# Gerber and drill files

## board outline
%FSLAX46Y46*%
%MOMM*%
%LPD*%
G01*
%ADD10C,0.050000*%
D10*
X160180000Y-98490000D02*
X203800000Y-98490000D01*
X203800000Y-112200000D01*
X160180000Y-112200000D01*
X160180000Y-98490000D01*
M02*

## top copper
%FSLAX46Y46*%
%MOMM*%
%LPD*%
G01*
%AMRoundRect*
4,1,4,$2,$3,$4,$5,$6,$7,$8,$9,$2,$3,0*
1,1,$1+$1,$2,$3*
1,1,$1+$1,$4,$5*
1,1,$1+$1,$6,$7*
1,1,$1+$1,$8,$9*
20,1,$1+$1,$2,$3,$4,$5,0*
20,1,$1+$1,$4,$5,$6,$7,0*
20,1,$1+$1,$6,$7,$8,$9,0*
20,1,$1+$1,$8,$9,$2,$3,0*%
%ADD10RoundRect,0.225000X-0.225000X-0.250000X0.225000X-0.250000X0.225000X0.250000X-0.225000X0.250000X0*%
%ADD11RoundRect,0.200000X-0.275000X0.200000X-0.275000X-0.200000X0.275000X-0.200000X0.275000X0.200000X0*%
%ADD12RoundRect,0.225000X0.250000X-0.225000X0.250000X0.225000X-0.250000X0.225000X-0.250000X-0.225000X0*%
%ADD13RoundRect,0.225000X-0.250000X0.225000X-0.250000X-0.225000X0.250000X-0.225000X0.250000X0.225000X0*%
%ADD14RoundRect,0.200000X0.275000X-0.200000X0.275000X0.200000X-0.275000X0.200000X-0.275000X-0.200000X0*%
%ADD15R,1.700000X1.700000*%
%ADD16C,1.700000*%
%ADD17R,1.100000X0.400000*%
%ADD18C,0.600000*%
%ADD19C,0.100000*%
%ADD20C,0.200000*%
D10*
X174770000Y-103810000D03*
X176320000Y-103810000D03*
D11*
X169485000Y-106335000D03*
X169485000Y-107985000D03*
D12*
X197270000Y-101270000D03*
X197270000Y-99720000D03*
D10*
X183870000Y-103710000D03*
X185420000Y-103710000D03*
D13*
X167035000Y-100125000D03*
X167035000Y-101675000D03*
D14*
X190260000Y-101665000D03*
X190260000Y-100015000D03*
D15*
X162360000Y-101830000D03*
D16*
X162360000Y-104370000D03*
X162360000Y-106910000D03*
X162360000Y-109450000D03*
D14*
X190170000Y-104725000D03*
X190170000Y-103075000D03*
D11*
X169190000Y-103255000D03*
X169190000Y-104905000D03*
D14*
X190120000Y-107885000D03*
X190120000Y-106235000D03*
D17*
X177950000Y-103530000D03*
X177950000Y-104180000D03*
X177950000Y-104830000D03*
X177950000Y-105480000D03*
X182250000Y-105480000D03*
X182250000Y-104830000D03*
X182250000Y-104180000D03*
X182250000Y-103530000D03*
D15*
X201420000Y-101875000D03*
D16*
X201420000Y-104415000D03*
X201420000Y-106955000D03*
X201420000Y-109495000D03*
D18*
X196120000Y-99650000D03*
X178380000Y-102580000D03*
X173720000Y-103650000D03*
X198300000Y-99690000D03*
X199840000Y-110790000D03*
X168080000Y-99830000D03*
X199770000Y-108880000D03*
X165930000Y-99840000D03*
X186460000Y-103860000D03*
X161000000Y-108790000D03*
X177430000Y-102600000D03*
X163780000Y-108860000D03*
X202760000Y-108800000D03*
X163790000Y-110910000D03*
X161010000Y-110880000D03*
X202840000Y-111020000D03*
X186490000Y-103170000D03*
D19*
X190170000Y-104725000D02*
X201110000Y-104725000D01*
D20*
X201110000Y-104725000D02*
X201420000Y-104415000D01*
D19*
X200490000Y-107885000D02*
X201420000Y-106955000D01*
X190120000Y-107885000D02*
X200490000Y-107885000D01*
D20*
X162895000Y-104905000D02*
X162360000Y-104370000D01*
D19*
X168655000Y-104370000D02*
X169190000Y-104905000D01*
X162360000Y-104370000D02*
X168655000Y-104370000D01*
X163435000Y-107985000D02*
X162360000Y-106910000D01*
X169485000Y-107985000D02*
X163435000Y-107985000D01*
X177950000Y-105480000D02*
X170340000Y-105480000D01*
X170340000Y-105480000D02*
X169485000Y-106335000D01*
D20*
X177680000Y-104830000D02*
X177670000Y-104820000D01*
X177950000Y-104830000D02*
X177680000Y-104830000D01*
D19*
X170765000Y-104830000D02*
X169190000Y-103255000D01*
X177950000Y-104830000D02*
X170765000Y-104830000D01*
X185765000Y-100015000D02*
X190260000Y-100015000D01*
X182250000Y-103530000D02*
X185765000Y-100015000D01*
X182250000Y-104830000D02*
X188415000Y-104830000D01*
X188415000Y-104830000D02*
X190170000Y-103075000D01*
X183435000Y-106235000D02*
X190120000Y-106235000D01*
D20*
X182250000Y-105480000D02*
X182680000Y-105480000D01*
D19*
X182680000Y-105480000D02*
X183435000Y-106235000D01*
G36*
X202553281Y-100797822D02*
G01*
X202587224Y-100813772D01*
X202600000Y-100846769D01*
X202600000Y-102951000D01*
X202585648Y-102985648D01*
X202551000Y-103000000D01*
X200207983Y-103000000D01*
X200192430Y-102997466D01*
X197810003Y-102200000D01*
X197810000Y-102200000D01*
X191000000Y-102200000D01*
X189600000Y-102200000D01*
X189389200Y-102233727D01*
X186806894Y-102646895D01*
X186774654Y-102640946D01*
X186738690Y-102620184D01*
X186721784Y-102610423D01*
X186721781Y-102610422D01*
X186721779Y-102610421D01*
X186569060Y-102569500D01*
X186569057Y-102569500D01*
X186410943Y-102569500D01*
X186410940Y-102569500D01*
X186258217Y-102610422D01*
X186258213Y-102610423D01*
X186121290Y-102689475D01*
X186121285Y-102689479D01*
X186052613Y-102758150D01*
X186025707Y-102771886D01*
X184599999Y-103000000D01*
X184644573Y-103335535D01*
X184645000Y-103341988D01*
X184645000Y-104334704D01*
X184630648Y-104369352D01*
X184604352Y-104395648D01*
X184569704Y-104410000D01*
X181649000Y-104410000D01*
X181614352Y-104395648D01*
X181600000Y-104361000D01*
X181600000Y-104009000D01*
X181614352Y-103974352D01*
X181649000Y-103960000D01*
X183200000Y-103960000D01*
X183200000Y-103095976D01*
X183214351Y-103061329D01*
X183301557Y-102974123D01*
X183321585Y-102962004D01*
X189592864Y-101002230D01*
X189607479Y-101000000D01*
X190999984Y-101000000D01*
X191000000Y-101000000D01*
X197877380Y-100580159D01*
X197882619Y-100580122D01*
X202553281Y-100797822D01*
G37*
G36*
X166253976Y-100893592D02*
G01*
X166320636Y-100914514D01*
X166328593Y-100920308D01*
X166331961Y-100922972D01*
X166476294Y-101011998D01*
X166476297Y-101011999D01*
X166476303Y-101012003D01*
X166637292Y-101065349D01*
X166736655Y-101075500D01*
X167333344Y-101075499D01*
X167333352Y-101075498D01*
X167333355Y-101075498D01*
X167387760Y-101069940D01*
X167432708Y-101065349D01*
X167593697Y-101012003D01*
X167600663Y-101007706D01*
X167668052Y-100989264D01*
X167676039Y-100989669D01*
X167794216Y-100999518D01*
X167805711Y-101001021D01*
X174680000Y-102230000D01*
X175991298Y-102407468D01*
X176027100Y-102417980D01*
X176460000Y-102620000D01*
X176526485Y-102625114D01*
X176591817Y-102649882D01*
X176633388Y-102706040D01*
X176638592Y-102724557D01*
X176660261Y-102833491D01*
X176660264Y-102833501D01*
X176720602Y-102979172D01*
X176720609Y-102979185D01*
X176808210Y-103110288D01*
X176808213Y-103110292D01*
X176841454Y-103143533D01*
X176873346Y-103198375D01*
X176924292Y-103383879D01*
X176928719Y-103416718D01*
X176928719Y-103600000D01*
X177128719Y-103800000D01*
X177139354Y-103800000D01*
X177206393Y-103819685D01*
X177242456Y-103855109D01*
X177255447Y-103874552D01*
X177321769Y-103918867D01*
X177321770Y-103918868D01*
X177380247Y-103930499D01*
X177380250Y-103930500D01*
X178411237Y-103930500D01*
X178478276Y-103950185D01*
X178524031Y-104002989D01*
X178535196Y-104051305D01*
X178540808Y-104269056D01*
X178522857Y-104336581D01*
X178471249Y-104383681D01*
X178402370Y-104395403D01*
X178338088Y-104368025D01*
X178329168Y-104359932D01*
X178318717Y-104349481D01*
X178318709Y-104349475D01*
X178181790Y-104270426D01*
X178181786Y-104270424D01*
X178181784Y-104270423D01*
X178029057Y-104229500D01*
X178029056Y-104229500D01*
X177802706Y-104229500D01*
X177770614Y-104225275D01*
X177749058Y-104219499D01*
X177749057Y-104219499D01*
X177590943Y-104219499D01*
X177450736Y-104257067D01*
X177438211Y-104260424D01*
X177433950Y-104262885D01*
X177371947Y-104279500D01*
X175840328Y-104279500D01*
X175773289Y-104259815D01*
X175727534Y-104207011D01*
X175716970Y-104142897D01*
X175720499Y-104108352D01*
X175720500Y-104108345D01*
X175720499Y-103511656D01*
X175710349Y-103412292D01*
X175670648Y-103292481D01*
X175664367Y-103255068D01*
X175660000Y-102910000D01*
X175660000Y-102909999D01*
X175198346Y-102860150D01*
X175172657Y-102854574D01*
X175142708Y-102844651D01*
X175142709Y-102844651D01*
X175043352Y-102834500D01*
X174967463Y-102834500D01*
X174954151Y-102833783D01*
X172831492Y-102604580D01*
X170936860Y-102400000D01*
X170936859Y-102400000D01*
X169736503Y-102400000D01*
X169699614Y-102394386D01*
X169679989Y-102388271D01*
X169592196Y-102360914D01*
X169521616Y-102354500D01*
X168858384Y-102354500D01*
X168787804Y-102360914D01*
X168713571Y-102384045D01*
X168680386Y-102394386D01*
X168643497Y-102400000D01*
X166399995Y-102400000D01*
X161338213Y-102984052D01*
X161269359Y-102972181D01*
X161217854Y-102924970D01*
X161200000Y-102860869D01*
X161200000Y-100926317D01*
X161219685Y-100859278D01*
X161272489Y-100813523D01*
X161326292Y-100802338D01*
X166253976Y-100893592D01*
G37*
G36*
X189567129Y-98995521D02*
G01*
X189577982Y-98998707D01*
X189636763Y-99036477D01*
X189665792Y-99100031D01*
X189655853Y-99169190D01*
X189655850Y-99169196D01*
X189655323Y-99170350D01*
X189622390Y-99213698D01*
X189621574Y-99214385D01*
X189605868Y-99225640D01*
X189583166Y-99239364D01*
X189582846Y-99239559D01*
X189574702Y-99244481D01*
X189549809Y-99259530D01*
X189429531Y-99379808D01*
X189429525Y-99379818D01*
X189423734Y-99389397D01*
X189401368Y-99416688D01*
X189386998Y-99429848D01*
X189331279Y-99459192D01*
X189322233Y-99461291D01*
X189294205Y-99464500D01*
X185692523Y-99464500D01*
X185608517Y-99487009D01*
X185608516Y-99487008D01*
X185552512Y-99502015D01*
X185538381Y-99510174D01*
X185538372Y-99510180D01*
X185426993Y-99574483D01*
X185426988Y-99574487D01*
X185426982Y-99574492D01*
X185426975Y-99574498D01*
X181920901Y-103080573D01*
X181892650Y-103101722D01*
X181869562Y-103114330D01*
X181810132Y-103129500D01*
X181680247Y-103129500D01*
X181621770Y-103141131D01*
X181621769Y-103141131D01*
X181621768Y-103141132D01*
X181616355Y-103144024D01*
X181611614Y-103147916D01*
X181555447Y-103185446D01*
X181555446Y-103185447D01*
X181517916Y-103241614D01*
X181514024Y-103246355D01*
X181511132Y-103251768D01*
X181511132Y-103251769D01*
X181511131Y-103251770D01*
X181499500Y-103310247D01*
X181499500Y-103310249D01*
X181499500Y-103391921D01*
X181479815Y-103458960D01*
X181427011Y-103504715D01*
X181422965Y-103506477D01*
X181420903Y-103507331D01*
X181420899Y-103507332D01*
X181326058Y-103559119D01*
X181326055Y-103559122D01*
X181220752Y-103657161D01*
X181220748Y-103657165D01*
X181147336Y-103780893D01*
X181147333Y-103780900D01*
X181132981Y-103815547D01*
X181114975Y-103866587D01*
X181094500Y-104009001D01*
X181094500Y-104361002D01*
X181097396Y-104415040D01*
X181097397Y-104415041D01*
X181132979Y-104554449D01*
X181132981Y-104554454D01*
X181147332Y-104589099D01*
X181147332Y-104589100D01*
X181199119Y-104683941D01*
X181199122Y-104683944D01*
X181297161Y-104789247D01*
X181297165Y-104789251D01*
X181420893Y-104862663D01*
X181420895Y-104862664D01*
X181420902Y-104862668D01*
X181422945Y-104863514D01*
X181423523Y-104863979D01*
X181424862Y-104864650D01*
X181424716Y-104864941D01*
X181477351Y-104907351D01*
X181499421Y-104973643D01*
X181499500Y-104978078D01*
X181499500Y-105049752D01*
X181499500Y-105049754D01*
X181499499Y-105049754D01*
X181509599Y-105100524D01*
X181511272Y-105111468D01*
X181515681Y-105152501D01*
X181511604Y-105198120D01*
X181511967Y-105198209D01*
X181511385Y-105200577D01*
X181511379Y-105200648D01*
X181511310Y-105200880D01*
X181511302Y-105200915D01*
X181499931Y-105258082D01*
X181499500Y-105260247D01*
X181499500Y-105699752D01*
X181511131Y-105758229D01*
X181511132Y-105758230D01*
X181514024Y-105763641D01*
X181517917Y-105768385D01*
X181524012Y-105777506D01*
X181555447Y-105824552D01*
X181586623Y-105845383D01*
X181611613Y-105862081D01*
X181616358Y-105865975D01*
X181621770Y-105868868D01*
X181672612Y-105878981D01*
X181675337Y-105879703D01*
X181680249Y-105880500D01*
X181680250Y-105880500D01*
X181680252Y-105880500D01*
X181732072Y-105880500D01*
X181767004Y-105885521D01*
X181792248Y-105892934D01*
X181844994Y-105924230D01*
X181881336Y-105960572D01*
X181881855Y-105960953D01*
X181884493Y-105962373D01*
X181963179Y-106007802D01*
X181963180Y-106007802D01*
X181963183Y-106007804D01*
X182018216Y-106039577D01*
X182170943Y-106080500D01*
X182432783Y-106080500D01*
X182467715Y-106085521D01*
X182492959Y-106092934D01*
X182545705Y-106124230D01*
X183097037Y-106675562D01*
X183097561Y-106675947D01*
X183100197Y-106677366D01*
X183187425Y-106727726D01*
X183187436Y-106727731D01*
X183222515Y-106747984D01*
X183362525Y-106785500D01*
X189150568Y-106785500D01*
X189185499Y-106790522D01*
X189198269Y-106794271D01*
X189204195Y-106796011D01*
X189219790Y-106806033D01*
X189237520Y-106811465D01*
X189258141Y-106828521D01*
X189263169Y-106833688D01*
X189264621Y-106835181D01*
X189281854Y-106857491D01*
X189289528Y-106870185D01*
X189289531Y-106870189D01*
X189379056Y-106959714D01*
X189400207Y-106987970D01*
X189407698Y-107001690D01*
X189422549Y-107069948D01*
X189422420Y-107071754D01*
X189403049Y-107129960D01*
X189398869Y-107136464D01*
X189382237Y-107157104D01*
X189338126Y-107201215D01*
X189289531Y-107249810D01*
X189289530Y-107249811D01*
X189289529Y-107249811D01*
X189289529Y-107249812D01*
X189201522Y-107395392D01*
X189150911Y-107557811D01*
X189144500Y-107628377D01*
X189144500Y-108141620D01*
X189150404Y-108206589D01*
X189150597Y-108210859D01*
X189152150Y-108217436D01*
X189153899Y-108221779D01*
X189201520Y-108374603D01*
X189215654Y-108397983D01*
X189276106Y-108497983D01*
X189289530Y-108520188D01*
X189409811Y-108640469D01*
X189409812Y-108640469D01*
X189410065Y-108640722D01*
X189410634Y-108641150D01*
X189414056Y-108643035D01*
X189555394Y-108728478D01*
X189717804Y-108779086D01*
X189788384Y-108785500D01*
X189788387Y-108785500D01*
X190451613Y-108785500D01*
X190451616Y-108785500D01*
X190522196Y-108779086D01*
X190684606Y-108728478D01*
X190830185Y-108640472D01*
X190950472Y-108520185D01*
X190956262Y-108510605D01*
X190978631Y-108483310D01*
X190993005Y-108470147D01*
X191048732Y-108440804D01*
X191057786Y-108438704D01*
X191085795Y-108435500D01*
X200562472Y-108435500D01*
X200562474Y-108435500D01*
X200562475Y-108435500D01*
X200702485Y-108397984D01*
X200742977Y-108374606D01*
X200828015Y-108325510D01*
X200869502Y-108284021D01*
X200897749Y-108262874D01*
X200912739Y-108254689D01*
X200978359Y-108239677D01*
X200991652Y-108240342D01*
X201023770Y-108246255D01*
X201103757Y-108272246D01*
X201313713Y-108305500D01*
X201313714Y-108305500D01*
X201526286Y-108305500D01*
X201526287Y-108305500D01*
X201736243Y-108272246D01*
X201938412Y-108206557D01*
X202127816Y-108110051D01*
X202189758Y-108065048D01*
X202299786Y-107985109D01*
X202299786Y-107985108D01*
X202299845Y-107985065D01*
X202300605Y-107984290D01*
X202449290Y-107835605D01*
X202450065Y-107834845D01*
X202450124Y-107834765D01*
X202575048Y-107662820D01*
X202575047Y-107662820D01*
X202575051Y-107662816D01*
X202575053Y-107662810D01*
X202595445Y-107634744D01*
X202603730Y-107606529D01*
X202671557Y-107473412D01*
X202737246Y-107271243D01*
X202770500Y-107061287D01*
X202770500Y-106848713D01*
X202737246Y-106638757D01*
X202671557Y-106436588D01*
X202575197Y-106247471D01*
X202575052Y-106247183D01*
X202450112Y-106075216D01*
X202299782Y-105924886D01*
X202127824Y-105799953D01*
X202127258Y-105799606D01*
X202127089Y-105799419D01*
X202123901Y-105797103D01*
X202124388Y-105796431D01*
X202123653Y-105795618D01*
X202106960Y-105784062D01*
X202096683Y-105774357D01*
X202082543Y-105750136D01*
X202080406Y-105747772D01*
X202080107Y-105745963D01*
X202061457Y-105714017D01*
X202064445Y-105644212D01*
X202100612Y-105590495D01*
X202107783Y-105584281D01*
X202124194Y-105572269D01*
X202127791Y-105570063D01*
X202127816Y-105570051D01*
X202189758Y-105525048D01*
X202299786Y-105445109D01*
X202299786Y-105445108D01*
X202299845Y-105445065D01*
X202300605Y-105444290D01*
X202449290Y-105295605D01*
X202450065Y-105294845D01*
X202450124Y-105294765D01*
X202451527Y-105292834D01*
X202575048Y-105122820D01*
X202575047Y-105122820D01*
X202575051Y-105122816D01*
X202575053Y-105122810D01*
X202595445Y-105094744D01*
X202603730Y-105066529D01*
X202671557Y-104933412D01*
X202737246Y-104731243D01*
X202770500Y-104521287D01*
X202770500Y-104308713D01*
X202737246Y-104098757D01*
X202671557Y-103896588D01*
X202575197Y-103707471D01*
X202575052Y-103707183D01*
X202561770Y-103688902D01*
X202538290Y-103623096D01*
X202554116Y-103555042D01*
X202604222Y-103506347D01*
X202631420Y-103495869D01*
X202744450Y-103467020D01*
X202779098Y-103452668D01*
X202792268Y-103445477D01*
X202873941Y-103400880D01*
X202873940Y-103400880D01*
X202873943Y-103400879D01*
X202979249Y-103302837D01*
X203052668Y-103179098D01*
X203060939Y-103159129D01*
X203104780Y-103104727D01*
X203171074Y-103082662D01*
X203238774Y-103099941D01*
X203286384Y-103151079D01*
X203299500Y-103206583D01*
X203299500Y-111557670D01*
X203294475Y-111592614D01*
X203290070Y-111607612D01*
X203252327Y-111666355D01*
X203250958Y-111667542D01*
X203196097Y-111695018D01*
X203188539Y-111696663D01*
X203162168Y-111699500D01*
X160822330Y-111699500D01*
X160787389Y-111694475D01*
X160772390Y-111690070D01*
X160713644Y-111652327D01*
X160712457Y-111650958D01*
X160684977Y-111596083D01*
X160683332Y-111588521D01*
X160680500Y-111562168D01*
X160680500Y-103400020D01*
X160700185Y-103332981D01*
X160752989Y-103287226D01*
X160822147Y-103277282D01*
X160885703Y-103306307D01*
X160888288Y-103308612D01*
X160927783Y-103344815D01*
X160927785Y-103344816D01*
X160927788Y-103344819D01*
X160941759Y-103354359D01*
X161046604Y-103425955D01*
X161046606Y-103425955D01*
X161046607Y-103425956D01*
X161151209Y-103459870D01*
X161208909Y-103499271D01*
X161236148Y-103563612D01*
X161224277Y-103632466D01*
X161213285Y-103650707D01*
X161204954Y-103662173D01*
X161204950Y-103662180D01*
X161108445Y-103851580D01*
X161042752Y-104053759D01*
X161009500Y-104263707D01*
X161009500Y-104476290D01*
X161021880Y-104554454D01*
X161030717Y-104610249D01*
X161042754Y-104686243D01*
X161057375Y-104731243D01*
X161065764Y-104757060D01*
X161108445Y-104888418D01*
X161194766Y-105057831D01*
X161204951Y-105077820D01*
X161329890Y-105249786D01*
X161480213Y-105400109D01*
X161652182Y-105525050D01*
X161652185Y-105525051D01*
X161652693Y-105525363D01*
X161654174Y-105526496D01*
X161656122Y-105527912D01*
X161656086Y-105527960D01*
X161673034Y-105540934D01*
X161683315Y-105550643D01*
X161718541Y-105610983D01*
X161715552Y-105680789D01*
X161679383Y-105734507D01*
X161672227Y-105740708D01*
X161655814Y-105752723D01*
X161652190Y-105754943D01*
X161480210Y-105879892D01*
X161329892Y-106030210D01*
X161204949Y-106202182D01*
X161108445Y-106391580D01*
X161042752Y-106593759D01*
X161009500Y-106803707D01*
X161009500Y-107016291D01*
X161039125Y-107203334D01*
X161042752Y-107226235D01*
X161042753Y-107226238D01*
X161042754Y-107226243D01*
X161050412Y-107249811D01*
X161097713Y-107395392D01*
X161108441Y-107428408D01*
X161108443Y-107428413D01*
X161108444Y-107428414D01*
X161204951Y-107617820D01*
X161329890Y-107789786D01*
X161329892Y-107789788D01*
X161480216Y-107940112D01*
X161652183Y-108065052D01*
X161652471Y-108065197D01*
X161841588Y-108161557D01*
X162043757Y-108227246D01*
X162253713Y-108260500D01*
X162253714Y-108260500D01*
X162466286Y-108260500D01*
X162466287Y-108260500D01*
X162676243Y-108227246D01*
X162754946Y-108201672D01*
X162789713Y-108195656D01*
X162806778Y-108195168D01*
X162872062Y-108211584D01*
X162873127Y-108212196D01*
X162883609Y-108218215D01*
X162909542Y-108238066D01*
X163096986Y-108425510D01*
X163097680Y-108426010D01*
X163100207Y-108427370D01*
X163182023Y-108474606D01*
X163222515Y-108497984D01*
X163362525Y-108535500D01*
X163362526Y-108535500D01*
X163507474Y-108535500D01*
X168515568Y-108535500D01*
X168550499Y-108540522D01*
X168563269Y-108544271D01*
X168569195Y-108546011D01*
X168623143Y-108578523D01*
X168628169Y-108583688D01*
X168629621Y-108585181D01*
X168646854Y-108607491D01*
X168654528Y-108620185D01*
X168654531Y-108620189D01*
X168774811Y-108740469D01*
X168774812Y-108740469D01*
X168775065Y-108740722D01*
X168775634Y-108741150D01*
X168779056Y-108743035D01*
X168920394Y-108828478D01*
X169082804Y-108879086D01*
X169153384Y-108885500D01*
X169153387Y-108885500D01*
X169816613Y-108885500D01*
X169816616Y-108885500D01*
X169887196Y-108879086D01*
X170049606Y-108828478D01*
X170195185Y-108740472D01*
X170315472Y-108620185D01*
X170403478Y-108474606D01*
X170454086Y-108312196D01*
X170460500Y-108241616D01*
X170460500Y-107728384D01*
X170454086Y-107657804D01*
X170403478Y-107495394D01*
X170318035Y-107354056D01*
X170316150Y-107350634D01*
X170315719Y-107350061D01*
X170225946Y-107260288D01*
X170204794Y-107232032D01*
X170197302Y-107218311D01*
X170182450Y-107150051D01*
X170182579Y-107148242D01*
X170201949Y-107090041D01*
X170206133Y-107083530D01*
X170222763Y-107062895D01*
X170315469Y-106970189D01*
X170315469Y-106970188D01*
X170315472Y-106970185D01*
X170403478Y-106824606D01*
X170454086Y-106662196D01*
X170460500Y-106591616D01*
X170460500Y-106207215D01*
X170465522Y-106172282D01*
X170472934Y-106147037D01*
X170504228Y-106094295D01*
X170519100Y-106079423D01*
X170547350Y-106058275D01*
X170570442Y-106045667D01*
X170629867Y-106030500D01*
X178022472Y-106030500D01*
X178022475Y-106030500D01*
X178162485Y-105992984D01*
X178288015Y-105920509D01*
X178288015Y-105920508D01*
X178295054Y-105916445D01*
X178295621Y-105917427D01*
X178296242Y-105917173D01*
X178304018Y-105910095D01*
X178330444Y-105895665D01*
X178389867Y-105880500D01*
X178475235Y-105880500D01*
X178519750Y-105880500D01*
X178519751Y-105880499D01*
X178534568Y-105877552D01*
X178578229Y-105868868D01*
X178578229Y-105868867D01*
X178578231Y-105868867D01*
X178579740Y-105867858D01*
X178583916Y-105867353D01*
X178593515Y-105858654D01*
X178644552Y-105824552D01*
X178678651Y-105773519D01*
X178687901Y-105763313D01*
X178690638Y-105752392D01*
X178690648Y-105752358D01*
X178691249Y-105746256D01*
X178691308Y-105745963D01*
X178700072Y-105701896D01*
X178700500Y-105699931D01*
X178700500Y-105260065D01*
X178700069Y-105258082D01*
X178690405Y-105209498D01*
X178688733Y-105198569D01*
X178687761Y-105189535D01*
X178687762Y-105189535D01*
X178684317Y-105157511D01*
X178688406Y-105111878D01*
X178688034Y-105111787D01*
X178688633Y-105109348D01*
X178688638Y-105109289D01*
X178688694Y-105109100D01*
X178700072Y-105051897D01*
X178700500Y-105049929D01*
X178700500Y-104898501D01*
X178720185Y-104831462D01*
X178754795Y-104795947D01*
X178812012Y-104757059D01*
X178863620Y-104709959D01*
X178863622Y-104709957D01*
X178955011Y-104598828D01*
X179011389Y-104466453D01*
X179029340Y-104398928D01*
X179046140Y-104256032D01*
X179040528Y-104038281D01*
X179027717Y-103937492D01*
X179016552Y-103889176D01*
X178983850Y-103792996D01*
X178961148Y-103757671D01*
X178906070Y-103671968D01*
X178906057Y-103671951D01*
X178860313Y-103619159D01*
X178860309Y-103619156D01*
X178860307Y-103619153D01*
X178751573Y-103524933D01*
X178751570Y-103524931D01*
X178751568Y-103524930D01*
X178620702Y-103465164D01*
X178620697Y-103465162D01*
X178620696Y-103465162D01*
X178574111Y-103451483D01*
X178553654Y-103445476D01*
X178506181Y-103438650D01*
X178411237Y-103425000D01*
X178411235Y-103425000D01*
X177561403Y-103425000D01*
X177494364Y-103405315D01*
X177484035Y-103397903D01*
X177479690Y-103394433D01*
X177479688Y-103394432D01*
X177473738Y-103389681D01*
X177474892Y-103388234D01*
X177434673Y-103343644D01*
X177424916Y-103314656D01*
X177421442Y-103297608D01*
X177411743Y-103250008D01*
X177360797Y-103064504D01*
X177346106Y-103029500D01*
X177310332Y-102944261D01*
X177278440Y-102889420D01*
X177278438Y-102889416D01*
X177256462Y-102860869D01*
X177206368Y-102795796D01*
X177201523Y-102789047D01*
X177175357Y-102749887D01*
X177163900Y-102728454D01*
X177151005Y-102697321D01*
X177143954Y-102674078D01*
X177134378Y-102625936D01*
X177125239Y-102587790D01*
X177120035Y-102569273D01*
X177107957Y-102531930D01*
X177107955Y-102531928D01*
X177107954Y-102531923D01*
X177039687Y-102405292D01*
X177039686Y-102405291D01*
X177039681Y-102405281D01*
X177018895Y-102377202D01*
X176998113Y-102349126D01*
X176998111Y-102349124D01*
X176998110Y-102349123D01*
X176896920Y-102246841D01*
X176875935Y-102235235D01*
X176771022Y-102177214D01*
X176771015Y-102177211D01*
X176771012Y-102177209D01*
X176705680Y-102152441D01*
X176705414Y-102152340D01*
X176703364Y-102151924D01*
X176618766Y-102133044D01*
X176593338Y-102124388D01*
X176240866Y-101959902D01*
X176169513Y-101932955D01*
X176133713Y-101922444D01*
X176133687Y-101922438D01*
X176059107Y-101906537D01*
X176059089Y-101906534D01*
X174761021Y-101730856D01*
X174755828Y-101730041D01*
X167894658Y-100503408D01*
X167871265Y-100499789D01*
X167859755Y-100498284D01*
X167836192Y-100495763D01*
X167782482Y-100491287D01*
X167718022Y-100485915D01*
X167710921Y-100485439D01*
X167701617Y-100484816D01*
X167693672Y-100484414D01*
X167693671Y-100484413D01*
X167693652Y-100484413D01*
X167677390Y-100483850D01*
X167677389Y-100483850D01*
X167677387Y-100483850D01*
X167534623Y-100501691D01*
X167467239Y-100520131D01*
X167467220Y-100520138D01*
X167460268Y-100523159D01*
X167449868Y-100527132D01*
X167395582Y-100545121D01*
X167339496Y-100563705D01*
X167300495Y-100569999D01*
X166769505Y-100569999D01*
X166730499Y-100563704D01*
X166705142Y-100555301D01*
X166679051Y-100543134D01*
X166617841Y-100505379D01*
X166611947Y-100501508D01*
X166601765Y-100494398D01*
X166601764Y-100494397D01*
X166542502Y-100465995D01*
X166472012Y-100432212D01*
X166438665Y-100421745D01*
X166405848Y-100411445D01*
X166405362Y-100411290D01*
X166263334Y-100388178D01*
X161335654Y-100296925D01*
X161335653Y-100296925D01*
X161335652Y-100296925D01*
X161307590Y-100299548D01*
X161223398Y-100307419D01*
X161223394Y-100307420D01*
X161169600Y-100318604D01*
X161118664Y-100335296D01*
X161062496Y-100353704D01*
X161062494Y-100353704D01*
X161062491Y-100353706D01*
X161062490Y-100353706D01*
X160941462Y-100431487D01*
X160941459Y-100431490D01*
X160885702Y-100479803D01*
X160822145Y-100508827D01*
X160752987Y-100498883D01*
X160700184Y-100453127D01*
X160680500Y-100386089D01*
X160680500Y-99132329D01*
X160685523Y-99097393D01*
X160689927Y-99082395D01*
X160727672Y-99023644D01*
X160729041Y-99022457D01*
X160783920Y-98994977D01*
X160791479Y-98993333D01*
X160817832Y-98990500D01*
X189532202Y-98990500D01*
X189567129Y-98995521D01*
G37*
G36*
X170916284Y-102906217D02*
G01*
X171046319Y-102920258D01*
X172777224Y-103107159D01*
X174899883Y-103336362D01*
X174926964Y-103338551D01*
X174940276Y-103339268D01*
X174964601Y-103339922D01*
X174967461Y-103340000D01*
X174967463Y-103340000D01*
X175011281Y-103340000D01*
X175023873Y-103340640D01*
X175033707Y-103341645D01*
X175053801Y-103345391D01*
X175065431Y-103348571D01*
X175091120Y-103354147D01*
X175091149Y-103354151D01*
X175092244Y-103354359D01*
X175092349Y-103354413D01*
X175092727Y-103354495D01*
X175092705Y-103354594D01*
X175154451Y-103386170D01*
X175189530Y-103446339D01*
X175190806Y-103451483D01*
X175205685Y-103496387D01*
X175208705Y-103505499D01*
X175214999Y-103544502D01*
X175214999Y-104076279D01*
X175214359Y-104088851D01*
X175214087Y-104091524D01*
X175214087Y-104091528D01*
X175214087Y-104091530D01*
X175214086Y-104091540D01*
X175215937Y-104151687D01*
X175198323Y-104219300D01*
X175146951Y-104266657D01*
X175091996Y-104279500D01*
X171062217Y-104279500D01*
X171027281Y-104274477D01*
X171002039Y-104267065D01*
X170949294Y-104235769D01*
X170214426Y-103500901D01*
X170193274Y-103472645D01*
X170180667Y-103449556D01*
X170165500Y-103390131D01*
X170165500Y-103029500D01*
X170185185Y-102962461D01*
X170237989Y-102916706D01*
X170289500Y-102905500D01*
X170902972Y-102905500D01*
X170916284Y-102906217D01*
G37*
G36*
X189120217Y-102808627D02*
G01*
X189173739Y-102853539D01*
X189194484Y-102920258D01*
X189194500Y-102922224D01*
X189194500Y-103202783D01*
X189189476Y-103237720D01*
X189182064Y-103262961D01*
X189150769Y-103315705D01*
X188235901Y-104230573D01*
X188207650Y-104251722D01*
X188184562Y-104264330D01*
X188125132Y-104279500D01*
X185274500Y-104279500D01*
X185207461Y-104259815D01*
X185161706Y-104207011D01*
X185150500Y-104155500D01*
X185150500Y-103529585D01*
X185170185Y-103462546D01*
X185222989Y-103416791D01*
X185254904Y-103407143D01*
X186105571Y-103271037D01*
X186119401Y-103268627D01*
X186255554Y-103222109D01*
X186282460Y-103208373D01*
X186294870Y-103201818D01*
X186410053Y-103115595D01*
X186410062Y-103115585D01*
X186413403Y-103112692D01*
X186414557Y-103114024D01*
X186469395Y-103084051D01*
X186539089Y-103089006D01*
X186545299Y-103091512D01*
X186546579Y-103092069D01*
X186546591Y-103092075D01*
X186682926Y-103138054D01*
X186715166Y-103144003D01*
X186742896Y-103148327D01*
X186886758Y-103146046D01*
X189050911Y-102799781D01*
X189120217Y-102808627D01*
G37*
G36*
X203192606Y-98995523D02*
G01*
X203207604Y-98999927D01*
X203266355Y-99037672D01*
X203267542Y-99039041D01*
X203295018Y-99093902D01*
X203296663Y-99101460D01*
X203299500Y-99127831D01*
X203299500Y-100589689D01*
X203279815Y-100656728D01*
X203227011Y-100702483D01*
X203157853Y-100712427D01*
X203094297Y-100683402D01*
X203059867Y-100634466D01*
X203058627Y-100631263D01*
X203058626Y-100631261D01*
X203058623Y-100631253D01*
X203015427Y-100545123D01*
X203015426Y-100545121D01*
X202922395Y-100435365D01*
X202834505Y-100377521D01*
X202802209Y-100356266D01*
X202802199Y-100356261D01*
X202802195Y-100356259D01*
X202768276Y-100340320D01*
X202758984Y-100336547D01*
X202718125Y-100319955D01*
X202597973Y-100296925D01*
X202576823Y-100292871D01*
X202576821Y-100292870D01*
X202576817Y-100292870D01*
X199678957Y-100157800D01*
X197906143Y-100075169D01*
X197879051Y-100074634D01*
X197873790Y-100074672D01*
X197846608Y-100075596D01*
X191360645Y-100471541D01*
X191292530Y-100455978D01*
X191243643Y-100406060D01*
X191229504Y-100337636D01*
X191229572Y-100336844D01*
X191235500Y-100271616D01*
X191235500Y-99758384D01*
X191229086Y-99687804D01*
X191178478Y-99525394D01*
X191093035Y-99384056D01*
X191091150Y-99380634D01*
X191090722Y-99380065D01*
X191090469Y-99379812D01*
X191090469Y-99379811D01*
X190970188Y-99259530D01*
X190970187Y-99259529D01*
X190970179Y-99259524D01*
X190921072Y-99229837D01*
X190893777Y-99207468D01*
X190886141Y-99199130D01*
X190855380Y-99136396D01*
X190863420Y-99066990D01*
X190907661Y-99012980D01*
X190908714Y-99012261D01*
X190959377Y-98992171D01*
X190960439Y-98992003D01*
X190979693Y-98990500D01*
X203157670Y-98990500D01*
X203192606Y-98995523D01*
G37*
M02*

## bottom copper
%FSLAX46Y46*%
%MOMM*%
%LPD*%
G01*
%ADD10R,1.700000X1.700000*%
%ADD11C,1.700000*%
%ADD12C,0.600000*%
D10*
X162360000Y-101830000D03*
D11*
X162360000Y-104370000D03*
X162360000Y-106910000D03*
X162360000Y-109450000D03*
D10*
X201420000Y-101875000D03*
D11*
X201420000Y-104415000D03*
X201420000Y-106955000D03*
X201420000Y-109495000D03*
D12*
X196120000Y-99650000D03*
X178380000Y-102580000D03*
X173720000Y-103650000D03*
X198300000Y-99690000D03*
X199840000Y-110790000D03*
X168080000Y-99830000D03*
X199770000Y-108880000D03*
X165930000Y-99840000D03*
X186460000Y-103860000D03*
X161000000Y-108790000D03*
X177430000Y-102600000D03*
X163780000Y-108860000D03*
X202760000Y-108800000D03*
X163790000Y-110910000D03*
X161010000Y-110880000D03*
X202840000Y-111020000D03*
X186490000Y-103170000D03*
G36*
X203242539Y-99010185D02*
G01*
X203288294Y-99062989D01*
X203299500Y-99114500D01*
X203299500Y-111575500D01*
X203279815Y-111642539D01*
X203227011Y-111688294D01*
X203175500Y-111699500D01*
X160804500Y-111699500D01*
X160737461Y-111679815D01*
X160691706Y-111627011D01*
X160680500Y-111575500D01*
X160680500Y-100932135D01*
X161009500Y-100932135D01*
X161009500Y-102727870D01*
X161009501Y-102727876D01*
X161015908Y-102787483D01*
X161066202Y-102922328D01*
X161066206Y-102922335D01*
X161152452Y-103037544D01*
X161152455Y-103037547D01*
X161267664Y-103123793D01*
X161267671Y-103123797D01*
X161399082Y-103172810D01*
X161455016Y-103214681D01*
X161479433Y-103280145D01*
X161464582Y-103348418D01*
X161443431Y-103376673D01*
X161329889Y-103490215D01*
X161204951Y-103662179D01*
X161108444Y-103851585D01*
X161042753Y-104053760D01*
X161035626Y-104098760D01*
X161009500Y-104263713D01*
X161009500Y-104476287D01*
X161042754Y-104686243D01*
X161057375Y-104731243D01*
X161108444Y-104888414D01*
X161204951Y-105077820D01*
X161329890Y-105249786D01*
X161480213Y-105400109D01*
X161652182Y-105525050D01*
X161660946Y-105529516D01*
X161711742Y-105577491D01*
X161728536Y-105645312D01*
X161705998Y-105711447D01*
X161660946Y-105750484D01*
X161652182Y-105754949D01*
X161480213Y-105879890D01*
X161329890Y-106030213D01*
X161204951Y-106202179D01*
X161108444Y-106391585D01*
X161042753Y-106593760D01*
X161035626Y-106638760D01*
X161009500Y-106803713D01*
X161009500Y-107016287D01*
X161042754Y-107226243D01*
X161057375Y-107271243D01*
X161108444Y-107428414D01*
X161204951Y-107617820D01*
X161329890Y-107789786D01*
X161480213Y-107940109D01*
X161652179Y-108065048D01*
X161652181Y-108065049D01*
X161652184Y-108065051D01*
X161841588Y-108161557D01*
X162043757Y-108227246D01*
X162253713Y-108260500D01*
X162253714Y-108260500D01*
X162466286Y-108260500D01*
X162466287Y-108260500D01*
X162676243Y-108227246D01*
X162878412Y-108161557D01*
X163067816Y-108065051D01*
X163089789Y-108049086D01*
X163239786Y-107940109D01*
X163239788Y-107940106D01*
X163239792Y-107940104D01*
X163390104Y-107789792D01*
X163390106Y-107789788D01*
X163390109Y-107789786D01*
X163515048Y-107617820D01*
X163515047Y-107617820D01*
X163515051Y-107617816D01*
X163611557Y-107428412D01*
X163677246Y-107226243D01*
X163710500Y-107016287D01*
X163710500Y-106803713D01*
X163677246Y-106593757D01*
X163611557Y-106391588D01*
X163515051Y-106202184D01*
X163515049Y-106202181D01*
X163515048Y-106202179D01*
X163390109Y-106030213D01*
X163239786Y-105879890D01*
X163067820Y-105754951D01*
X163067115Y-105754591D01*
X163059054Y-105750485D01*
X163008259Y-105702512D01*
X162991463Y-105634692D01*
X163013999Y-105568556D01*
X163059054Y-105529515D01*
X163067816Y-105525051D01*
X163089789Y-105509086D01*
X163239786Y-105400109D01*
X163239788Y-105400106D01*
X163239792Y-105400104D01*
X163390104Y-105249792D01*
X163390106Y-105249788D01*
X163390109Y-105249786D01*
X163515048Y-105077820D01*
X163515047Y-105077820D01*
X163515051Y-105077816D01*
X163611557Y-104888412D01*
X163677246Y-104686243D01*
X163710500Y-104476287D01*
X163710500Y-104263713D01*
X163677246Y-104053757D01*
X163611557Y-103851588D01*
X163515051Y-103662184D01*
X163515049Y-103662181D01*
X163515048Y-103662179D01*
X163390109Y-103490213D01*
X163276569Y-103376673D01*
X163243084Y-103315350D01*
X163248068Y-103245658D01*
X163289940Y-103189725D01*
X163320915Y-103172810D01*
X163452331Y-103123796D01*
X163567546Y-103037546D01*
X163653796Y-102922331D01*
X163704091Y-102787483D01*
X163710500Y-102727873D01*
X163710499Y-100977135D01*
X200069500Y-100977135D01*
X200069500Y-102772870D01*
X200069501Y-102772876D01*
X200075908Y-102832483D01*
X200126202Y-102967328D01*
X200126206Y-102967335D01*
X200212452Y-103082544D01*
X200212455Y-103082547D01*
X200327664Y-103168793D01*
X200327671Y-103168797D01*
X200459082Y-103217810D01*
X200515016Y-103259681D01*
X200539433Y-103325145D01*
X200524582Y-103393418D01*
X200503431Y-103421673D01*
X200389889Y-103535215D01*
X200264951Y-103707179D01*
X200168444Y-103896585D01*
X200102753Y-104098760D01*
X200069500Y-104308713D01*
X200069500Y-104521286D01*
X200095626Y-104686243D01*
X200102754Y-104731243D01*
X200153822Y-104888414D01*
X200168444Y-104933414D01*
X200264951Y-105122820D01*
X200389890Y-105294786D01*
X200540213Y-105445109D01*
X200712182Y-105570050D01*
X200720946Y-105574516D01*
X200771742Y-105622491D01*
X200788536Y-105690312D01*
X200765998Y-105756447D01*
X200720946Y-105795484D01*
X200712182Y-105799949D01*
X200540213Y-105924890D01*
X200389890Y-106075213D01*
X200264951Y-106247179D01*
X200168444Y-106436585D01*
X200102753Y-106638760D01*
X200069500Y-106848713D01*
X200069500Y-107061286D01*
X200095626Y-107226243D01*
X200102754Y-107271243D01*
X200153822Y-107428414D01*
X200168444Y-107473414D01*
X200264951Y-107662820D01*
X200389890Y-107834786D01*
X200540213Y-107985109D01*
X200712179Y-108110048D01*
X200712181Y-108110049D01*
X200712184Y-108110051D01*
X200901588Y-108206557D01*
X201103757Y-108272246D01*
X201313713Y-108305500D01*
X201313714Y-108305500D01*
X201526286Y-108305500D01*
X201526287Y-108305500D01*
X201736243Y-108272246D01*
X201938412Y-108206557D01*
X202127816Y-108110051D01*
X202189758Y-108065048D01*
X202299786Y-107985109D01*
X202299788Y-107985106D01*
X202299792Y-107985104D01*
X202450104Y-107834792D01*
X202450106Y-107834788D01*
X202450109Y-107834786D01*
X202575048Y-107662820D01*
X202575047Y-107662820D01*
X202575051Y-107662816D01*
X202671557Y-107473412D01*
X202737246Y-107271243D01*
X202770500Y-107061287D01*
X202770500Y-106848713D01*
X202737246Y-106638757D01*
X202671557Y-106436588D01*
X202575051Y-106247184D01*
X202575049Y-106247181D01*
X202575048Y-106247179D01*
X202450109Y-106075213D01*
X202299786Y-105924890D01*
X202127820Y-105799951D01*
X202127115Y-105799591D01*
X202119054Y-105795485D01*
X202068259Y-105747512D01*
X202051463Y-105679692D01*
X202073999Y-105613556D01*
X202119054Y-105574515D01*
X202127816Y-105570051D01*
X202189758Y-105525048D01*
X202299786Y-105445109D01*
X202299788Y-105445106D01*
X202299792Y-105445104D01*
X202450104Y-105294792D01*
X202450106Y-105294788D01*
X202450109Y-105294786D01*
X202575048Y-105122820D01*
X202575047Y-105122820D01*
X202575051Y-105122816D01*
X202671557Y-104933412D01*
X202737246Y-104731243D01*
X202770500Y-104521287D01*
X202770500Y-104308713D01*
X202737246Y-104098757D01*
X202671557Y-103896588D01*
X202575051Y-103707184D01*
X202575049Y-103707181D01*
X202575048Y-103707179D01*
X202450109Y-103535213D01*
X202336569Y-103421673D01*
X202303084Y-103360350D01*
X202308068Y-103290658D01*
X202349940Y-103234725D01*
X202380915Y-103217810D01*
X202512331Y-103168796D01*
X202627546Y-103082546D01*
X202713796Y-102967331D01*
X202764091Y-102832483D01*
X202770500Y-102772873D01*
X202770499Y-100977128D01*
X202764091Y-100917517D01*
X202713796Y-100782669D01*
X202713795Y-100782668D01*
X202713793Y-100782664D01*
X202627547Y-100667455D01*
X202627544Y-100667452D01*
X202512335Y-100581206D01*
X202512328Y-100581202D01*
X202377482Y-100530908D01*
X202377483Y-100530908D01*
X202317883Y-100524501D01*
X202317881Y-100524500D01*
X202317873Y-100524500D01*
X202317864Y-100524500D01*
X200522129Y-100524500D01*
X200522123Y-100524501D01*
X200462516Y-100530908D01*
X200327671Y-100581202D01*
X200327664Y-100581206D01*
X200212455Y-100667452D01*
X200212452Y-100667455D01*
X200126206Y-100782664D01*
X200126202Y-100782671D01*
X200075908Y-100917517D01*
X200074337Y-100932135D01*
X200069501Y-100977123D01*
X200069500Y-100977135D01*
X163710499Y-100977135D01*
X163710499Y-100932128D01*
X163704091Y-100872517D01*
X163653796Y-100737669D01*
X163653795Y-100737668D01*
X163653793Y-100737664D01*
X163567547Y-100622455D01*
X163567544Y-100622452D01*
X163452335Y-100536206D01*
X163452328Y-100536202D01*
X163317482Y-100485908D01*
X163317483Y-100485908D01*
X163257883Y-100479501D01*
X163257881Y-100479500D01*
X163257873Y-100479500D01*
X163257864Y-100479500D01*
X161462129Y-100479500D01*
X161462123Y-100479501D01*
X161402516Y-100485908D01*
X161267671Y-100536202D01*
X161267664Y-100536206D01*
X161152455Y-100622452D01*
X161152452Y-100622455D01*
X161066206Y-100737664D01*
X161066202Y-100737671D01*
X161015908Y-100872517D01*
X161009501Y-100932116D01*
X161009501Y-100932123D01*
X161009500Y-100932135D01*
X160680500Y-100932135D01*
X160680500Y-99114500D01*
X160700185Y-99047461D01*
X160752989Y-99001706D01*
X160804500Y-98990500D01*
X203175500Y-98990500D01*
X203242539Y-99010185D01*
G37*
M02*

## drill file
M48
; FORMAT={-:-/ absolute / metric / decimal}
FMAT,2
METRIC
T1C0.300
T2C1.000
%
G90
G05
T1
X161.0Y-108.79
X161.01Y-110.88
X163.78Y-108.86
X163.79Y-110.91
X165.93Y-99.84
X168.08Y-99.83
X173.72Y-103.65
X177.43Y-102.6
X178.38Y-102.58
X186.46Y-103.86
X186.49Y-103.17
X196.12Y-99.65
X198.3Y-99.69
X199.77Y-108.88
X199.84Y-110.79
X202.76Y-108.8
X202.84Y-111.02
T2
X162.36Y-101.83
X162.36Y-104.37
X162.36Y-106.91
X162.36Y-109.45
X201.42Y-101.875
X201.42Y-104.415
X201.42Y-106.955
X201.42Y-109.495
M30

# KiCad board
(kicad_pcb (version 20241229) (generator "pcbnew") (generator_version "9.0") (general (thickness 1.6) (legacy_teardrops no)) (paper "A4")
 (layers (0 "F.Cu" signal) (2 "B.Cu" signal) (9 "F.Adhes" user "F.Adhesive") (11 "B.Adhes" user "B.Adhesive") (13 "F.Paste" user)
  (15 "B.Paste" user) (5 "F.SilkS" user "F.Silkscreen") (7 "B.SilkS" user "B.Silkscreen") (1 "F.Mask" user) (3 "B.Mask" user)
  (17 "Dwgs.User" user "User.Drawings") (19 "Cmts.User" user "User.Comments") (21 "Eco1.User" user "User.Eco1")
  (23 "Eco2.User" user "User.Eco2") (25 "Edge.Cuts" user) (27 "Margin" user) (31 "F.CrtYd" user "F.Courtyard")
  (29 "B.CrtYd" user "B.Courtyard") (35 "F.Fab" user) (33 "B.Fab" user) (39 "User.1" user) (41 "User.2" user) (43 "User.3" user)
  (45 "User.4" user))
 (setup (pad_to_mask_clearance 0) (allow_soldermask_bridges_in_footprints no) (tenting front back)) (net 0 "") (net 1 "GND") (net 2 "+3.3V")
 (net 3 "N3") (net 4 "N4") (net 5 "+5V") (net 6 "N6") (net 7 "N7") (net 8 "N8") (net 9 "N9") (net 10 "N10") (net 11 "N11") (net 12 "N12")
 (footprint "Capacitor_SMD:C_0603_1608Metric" (layer "F.Cu") (at 175.545 103.81)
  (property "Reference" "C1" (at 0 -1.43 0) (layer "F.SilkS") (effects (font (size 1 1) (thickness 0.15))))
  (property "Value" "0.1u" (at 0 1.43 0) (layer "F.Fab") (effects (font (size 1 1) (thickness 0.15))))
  (pad "1" smd roundrect (at -0.775 0) (size 0.9 0.95) (layers "F.Cu" "F.Mask" "F.Paste") (roundrect_rratio 0.25) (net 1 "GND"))
  (pad "2" smd roundrect (at 0.775 0) (size 0.9 0.95) (layers "F.Cu" "F.Mask" "F.Paste") (roundrect_rratio 0.25) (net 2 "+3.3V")))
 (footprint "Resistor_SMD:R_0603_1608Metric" (layer "F.Cu") (at 169.485 107.16 -90)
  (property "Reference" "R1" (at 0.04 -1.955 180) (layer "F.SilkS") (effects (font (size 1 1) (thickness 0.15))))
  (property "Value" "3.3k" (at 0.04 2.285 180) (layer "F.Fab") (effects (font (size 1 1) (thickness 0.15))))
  (pad "1" smd roundrect (at -0.825 0 270) (size 0.8 0.95) (layers "F.Cu" "F.Mask" "F.Paste") (roundrect_rratio 0.25) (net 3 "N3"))
  (pad "2" smd roundrect (at 0.825 0 270) (size 0.8 0.95) (layers "F.Cu" "F.Mask" "F.Paste") (roundrect_rratio 0.25) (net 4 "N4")))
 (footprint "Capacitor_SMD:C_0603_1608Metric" (layer "F.Cu") (at 197.27 100.495 90)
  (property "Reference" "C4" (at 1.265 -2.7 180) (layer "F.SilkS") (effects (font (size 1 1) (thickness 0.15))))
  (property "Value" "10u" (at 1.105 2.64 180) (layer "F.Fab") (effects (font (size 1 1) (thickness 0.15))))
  (pad "1" smd roundrect (at -0.775 0 90) (size 0.9 0.95) (layers "F.Cu" "F.Mask" "F.Paste") (roundrect_rratio 0.25) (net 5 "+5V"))
  (pad "2" smd roundrect (at 0.775 0 90) (size 0.9 0.95) (layers "F.Cu" "F.Mask" "F.Paste") (roundrect_rratio 0.25) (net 1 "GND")))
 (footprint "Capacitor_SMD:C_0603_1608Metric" (layer "F.Cu") (at 184.645 103.71)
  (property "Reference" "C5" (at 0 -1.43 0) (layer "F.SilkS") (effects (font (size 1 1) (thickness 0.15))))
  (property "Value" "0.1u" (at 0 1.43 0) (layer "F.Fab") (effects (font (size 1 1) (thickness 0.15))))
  (pad "1" smd roundrect (at -0.775 0) (size 0.9 0.95) (layers "F.Cu" "F.Mask" "F.Paste") (roundrect_rratio 0.25) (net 5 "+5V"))
  (pad "2" smd roundrect (at 0.775 0) (size 0.9 0.95) (layers "F.Cu" "F.Mask" "F.Paste") (roundrect_rratio 0.25) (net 1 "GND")))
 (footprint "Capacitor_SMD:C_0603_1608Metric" (layer "F.Cu") (at 167.035 100.9 -90)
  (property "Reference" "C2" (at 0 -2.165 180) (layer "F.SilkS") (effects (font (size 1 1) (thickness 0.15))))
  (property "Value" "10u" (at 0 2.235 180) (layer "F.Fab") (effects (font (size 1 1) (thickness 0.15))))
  (pad "1" smd roundrect (at -0.775 0 270) (size 0.9 0.95) (layers "F.Cu" "F.Mask" "F.Paste") (roundrect_rratio 0.25) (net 1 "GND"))
  (pad "2" smd roundrect (at 0.775 0 270) (size 0.9 0.95) (layers "F.Cu" "F.Mask" "F.Paste") (roundrect_rratio 0.25) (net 2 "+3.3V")))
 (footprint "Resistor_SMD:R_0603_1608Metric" (layer "F.Cu") (at 190.26 100.84 90)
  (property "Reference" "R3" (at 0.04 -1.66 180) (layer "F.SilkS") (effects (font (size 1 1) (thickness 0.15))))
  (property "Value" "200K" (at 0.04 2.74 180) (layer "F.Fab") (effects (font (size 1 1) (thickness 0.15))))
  (pad "1" smd roundrect (at -0.825 0 90) (size 0.8 0.95) (layers "F.Cu" "F.Mask" "F.Paste") (roundrect_rratio 0.25) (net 5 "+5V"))
  (pad "2" smd roundrect (at 0.825 0 90) (size 0.8 0.95) (layers "F.Cu" "F.Mask" "F.Paste") (roundrect_rratio 0.25) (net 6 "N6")))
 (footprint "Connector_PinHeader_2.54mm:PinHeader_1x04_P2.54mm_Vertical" (layer "F.Cu") (at 162.36 101.83)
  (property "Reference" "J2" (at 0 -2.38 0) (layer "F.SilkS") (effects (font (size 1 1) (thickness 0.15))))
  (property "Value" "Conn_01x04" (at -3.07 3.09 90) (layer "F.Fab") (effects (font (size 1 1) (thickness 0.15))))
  (pad "1" thru_hole rect (at 0 0) (size 1.7 1.7) (drill 1) (layers "*.Cu" "*.Mask") (remove_unused_layers no) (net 2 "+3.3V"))
  (pad "2" thru_hole circle (at 0 2.54) (size 1.7 1.7) (drill 1) (layers "*.Cu" "*.Mask") (remove_unused_layers no) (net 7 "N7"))
  (pad "3" thru_hole circle (at 0 5.08) (size 1.7 1.7) (drill 1) (layers "*.Cu" "*.Mask") (remove_unused_layers no) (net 4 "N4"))
  (pad "4" thru_hole circle (at 0 7.62) (size 1.7 1.7) (drill 1) (layers "*.Cu" "*.Mask") (remove_unused_layers no) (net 1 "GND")))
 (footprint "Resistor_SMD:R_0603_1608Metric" (layer "F.Cu") (at 190.17 103.9 90)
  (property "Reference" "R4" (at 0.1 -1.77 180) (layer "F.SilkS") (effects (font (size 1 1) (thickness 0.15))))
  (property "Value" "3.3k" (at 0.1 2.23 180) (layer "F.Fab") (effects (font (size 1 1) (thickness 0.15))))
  (pad "1" smd roundrect (at -0.825 0 90) (size 0.8 0.95) (layers "F.Cu" "F.Mask" "F.Paste") (roundrect_rratio 0.25) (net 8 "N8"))
  (pad "2" smd roundrect (at 0.825 0 90) (size 0.8 0.95) (layers "F.Cu" "F.Mask" "F.Paste") (roundrect_rratio 0.25) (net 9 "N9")))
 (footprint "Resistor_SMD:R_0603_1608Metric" (layer "F.Cu") (at 169.19 104.08 -90)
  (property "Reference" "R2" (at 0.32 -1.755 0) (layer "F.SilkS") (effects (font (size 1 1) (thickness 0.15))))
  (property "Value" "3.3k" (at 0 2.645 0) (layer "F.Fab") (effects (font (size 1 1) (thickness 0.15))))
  (pad "1" smd roundrect (at -0.825 0 270) (size 0.8 0.95) (layers "F.Cu" "F.Mask" "F.Paste") (roundrect_rratio 0.25) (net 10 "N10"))
  (pad "2" smd roundrect (at 0.825 0 270) (size 0.8 0.95) (layers "F.Cu" "F.Mask" "F.Paste") (roundrect_rratio 0.25) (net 7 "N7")))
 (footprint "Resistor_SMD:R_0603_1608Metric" (layer "F.Cu") (at 190.12 107.06 90)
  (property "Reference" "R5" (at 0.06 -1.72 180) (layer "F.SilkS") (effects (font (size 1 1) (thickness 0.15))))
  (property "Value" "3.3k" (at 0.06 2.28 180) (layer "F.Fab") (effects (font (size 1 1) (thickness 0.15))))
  (pad "1" smd roundrect (at -0.825 0 90) (size 0.8 0.95) (layers "F.Cu" "F.Mask" "F.Paste") (roundrect_rratio 0.25) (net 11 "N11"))
  (pad "2" smd roundrect (at 0.825 0 90) (size 0.8 0.95) (layers "F.Cu" "F.Mask" "F.Paste") (roundrect_rratio 0.25) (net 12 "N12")))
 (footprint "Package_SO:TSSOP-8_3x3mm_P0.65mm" (layer "F.Cu") (at 180.1 104.505)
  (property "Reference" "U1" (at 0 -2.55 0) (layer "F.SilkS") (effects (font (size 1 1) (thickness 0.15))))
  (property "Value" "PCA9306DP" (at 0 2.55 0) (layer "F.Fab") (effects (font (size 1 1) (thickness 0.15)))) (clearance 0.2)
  (pad "1" smd rect (at -2.15 -0.975) (size 1.1 0.4) (layers "F.Cu" "F.Mask" "F.Paste") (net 1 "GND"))
  (pad "2" smd rect (at -2.15 -0.325) (size 1.1 0.4) (layers "F.Cu" "F.Mask" "F.Paste") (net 2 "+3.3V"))
  (pad "3" smd rect (at -2.15 0.325) (size 1.1 0.4) (layers "F.Cu" "F.Mask" "F.Paste") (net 10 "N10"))
  (pad "4" smd rect (at -2.15 0.975) (size 1.1 0.4) (layers "F.Cu" "F.Mask" "F.Paste") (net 3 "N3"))
  (pad "5" smd rect (at 2.15 0.975) (size 1.1 0.4) (layers "F.Cu" "F.Mask" "F.Paste") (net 12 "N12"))
  (pad "6" smd rect (at 2.15 0.325) (size 1.1 0.4) (layers "F.Cu" "F.Mask" "F.Paste") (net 9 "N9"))
  (pad "7" smd rect (at 2.15 -0.325) (size 1.1 0.4) (layers "F.Cu" "F.Mask" "F.Paste") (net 5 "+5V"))
  (pad "8" smd rect (at 2.15 -0.975) (size 1.1 0.4) (layers "F.Cu" "F.Mask" "F.Paste") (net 6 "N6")))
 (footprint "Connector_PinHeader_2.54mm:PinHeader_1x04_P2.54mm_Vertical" (layer "F.Cu") (at 201.42 101.875)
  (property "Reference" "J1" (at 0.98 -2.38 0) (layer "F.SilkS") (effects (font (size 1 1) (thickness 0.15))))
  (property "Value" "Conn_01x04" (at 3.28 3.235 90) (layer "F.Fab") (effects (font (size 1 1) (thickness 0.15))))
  (pad "1" thru_hole rect (at 0 0) (size 1.7 1.7) (drill 1) (layers "*.Cu" "*.Mask") (remove_unused_layers no) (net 5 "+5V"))
  (pad "2" thru_hole circle (at 0 2.54) (size 1.7 1.7) (drill 1) (layers "*.Cu" "*.Mask") (remove_unused_layers no) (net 8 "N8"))
  (pad "3" thru_hole circle (at 0 5.08) (size 1.7 1.7) (drill 1) (layers "*.Cu" "*.Mask") (remove_unused_layers no) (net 11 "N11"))
  (pad "4" thru_hole circle (at 0 7.62) (size 1.7 1.7) (drill 1) (layers "*.Cu" "*.Mask") (remove_unused_layers no) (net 1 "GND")))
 (gr_rect (start 160.18 98.49) (end 203.8 112.2) (stroke (width 0.05) (type default)) (fill no) (layer "Edge.Cuts"))
 (via (at 196.12 99.65) (size 0.6) (drill 0.3) (layers "F.Cu" "B.Cu") (free yes) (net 1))
 (via (at 178.38 102.58) (size 0.6) (drill 0.3) (layers "F.Cu" "B.Cu") (free yes) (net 1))
 (via (at 173.72 103.65) (size 0.6) (drill 0.3) (layers "F.Cu" "B.Cu") (free yes) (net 1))
 (via (at 198.3 99.69) (size 0.6) (drill 0.3) (layers "F.Cu" "B.Cu") (free yes) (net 1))
 (via (at 199.84 110.79) (size 0.6) (drill 0.3) (layers "F.Cu" "B.Cu") (free yes) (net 1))
 (via (at 168.08 99.83) (size 0.6) (drill 0.3) (layers "F.Cu" "B.Cu") (free yes) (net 1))
 (via (at 199.77 108.88) (size 0.6) (drill 0.3) (layers "F.Cu" "B.Cu") (free yes) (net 1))
 (via (at 165.93 99.84) (size 0.6) (drill 0.3) (layers "F.Cu" "B.Cu") (free yes) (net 1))
 (via (at 186.46 103.86) (size 0.6) (drill 0.3) (layers "F.Cu" "B.Cu") (free yes) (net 1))
 (via (at 161 108.79) (size 0.6) (drill 0.3) (layers "F.Cu" "B.Cu") (free yes) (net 1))
 (via (at 177.43 102.6) (size 0.6) (drill 0.3) (layers "F.Cu" "B.Cu") (free yes) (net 1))
 (via (at 163.78 108.86) (size 0.6) (drill 0.3) (layers "F.Cu" "B.Cu") (free yes) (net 1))
 (via (at 202.76 108.8) (size 0.6) (drill 0.3) (layers "F.Cu" "B.Cu") (free yes) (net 1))
 (via (at 163.79 110.91) (size 0.6) (drill 0.3) (layers "F.Cu" "B.Cu") (free yes) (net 1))
 (via (at 161.01 110.88) (size 0.6) (drill 0.3) (layers "F.Cu" "B.Cu") (free yes) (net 1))
 (via (at 202.84 111.02) (size 0.6) (drill 0.3) (layers "F.Cu" "B.Cu") (free yes) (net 1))
 (via (at 186.49 103.17) (size 0.6) (drill 0.3) (layers "F.Cu" "B.Cu") (free yes) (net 1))
 (segment (start 190.17 104.725) (end 201.11 104.725) (width 0.1) (layer "F.Cu") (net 8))
 (segment (start 201.11 104.725) (end 201.42 104.415) (width 0.2) (layer "F.Cu") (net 8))
 (segment (start 200.49 107.885) (end 201.42 106.955) (width 0.1) (layer "F.Cu") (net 11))
 (segment (start 190.12 107.885) (end 200.49 107.885) (width 0.1) (layer "F.Cu") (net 11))
 (segment (start 162.895 104.905) (end 162.36 104.37) (width 0.2) (layer "F.Cu") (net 7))
 (segment (start 168.655 104.37) (end 169.19 104.905) (width 0.1) (layer "F.Cu") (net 7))
 (segment (start 162.36 104.37) (end 168.655 104.37) (width 0.1) (layer "F.Cu") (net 7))
 (segment (start 163.435 107.985) (end 162.36 106.91) (width 0.1) (layer "F.Cu") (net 4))
 (segment (start 169.485 107.985) (end 163.435 107.985) (width 0.1) (layer "F.Cu") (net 4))
 (segment (start 177.95 105.48) (end 170.34 105.48) (width 0.1) (layer "F.Cu") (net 3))
 (segment (start 170.34 105.48) (end 169.485 106.335) (width 0.1) (layer "F.Cu") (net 3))
 (segment (start 177.68 104.83) (end 177.67 104.82) (width 0.2) (layer "F.Cu") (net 10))
 (segment (start 177.95 104.83) (end 177.68 104.83) (width 0.2) (layer "F.Cu") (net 10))
 (segment (start 170.765 104.83) (end 169.19 103.255) (width 0.1) (layer "F.Cu") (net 10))
 (segment (start 177.95 104.83) (end 170.765 104.83) (width 0.1) (layer "F.Cu") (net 10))
 (segment (start 185.765 100.015) (end 190.26 100.015) (width 0.1) (layer "F.Cu") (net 6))
 (segment (start 182.25 103.53) (end 185.765 100.015) (width 0.1) (layer "F.Cu") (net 6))
 (segment (start 182.25 104.83) (end 188.415 104.83) (width 0.1) (layer "F.Cu") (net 9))
 (segment (start 188.415 104.83) (end 190.17 103.075) (width 0.1) (layer "F.Cu") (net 9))
 (segment (start 183.435 106.235) (end 190.12 106.235) (width 0.1) (layer "F.Cu") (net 12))
 (segment (start 182.25 105.48) (end 182.68 105.48) (width 0.2) (layer "F.Cu") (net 12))
 (segment (start 182.68 105.48) (end 183.435 106.235) (width 0.1) (layer "F.Cu") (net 12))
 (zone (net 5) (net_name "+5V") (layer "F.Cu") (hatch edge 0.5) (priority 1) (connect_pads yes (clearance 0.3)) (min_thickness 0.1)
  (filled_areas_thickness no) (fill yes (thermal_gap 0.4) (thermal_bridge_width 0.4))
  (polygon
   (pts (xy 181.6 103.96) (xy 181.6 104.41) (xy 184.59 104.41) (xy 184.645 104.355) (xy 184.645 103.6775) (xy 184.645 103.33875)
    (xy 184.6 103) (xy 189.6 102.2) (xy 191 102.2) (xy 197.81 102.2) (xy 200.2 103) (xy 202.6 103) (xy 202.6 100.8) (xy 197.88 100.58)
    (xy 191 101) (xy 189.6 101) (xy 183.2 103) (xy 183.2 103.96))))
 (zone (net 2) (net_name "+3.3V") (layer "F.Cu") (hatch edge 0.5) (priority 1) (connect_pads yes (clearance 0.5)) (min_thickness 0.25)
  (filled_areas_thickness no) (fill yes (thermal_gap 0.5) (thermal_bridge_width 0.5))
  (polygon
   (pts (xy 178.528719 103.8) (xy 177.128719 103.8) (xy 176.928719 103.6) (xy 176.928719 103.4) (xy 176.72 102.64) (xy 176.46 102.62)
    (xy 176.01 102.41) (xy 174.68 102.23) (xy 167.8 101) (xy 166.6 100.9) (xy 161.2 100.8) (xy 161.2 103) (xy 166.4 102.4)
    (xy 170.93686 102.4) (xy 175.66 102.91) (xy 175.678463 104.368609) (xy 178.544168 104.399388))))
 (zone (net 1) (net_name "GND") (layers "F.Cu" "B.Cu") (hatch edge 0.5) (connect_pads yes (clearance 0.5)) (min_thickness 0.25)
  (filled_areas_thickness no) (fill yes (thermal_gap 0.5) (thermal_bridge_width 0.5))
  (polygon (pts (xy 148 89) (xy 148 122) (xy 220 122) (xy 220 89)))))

